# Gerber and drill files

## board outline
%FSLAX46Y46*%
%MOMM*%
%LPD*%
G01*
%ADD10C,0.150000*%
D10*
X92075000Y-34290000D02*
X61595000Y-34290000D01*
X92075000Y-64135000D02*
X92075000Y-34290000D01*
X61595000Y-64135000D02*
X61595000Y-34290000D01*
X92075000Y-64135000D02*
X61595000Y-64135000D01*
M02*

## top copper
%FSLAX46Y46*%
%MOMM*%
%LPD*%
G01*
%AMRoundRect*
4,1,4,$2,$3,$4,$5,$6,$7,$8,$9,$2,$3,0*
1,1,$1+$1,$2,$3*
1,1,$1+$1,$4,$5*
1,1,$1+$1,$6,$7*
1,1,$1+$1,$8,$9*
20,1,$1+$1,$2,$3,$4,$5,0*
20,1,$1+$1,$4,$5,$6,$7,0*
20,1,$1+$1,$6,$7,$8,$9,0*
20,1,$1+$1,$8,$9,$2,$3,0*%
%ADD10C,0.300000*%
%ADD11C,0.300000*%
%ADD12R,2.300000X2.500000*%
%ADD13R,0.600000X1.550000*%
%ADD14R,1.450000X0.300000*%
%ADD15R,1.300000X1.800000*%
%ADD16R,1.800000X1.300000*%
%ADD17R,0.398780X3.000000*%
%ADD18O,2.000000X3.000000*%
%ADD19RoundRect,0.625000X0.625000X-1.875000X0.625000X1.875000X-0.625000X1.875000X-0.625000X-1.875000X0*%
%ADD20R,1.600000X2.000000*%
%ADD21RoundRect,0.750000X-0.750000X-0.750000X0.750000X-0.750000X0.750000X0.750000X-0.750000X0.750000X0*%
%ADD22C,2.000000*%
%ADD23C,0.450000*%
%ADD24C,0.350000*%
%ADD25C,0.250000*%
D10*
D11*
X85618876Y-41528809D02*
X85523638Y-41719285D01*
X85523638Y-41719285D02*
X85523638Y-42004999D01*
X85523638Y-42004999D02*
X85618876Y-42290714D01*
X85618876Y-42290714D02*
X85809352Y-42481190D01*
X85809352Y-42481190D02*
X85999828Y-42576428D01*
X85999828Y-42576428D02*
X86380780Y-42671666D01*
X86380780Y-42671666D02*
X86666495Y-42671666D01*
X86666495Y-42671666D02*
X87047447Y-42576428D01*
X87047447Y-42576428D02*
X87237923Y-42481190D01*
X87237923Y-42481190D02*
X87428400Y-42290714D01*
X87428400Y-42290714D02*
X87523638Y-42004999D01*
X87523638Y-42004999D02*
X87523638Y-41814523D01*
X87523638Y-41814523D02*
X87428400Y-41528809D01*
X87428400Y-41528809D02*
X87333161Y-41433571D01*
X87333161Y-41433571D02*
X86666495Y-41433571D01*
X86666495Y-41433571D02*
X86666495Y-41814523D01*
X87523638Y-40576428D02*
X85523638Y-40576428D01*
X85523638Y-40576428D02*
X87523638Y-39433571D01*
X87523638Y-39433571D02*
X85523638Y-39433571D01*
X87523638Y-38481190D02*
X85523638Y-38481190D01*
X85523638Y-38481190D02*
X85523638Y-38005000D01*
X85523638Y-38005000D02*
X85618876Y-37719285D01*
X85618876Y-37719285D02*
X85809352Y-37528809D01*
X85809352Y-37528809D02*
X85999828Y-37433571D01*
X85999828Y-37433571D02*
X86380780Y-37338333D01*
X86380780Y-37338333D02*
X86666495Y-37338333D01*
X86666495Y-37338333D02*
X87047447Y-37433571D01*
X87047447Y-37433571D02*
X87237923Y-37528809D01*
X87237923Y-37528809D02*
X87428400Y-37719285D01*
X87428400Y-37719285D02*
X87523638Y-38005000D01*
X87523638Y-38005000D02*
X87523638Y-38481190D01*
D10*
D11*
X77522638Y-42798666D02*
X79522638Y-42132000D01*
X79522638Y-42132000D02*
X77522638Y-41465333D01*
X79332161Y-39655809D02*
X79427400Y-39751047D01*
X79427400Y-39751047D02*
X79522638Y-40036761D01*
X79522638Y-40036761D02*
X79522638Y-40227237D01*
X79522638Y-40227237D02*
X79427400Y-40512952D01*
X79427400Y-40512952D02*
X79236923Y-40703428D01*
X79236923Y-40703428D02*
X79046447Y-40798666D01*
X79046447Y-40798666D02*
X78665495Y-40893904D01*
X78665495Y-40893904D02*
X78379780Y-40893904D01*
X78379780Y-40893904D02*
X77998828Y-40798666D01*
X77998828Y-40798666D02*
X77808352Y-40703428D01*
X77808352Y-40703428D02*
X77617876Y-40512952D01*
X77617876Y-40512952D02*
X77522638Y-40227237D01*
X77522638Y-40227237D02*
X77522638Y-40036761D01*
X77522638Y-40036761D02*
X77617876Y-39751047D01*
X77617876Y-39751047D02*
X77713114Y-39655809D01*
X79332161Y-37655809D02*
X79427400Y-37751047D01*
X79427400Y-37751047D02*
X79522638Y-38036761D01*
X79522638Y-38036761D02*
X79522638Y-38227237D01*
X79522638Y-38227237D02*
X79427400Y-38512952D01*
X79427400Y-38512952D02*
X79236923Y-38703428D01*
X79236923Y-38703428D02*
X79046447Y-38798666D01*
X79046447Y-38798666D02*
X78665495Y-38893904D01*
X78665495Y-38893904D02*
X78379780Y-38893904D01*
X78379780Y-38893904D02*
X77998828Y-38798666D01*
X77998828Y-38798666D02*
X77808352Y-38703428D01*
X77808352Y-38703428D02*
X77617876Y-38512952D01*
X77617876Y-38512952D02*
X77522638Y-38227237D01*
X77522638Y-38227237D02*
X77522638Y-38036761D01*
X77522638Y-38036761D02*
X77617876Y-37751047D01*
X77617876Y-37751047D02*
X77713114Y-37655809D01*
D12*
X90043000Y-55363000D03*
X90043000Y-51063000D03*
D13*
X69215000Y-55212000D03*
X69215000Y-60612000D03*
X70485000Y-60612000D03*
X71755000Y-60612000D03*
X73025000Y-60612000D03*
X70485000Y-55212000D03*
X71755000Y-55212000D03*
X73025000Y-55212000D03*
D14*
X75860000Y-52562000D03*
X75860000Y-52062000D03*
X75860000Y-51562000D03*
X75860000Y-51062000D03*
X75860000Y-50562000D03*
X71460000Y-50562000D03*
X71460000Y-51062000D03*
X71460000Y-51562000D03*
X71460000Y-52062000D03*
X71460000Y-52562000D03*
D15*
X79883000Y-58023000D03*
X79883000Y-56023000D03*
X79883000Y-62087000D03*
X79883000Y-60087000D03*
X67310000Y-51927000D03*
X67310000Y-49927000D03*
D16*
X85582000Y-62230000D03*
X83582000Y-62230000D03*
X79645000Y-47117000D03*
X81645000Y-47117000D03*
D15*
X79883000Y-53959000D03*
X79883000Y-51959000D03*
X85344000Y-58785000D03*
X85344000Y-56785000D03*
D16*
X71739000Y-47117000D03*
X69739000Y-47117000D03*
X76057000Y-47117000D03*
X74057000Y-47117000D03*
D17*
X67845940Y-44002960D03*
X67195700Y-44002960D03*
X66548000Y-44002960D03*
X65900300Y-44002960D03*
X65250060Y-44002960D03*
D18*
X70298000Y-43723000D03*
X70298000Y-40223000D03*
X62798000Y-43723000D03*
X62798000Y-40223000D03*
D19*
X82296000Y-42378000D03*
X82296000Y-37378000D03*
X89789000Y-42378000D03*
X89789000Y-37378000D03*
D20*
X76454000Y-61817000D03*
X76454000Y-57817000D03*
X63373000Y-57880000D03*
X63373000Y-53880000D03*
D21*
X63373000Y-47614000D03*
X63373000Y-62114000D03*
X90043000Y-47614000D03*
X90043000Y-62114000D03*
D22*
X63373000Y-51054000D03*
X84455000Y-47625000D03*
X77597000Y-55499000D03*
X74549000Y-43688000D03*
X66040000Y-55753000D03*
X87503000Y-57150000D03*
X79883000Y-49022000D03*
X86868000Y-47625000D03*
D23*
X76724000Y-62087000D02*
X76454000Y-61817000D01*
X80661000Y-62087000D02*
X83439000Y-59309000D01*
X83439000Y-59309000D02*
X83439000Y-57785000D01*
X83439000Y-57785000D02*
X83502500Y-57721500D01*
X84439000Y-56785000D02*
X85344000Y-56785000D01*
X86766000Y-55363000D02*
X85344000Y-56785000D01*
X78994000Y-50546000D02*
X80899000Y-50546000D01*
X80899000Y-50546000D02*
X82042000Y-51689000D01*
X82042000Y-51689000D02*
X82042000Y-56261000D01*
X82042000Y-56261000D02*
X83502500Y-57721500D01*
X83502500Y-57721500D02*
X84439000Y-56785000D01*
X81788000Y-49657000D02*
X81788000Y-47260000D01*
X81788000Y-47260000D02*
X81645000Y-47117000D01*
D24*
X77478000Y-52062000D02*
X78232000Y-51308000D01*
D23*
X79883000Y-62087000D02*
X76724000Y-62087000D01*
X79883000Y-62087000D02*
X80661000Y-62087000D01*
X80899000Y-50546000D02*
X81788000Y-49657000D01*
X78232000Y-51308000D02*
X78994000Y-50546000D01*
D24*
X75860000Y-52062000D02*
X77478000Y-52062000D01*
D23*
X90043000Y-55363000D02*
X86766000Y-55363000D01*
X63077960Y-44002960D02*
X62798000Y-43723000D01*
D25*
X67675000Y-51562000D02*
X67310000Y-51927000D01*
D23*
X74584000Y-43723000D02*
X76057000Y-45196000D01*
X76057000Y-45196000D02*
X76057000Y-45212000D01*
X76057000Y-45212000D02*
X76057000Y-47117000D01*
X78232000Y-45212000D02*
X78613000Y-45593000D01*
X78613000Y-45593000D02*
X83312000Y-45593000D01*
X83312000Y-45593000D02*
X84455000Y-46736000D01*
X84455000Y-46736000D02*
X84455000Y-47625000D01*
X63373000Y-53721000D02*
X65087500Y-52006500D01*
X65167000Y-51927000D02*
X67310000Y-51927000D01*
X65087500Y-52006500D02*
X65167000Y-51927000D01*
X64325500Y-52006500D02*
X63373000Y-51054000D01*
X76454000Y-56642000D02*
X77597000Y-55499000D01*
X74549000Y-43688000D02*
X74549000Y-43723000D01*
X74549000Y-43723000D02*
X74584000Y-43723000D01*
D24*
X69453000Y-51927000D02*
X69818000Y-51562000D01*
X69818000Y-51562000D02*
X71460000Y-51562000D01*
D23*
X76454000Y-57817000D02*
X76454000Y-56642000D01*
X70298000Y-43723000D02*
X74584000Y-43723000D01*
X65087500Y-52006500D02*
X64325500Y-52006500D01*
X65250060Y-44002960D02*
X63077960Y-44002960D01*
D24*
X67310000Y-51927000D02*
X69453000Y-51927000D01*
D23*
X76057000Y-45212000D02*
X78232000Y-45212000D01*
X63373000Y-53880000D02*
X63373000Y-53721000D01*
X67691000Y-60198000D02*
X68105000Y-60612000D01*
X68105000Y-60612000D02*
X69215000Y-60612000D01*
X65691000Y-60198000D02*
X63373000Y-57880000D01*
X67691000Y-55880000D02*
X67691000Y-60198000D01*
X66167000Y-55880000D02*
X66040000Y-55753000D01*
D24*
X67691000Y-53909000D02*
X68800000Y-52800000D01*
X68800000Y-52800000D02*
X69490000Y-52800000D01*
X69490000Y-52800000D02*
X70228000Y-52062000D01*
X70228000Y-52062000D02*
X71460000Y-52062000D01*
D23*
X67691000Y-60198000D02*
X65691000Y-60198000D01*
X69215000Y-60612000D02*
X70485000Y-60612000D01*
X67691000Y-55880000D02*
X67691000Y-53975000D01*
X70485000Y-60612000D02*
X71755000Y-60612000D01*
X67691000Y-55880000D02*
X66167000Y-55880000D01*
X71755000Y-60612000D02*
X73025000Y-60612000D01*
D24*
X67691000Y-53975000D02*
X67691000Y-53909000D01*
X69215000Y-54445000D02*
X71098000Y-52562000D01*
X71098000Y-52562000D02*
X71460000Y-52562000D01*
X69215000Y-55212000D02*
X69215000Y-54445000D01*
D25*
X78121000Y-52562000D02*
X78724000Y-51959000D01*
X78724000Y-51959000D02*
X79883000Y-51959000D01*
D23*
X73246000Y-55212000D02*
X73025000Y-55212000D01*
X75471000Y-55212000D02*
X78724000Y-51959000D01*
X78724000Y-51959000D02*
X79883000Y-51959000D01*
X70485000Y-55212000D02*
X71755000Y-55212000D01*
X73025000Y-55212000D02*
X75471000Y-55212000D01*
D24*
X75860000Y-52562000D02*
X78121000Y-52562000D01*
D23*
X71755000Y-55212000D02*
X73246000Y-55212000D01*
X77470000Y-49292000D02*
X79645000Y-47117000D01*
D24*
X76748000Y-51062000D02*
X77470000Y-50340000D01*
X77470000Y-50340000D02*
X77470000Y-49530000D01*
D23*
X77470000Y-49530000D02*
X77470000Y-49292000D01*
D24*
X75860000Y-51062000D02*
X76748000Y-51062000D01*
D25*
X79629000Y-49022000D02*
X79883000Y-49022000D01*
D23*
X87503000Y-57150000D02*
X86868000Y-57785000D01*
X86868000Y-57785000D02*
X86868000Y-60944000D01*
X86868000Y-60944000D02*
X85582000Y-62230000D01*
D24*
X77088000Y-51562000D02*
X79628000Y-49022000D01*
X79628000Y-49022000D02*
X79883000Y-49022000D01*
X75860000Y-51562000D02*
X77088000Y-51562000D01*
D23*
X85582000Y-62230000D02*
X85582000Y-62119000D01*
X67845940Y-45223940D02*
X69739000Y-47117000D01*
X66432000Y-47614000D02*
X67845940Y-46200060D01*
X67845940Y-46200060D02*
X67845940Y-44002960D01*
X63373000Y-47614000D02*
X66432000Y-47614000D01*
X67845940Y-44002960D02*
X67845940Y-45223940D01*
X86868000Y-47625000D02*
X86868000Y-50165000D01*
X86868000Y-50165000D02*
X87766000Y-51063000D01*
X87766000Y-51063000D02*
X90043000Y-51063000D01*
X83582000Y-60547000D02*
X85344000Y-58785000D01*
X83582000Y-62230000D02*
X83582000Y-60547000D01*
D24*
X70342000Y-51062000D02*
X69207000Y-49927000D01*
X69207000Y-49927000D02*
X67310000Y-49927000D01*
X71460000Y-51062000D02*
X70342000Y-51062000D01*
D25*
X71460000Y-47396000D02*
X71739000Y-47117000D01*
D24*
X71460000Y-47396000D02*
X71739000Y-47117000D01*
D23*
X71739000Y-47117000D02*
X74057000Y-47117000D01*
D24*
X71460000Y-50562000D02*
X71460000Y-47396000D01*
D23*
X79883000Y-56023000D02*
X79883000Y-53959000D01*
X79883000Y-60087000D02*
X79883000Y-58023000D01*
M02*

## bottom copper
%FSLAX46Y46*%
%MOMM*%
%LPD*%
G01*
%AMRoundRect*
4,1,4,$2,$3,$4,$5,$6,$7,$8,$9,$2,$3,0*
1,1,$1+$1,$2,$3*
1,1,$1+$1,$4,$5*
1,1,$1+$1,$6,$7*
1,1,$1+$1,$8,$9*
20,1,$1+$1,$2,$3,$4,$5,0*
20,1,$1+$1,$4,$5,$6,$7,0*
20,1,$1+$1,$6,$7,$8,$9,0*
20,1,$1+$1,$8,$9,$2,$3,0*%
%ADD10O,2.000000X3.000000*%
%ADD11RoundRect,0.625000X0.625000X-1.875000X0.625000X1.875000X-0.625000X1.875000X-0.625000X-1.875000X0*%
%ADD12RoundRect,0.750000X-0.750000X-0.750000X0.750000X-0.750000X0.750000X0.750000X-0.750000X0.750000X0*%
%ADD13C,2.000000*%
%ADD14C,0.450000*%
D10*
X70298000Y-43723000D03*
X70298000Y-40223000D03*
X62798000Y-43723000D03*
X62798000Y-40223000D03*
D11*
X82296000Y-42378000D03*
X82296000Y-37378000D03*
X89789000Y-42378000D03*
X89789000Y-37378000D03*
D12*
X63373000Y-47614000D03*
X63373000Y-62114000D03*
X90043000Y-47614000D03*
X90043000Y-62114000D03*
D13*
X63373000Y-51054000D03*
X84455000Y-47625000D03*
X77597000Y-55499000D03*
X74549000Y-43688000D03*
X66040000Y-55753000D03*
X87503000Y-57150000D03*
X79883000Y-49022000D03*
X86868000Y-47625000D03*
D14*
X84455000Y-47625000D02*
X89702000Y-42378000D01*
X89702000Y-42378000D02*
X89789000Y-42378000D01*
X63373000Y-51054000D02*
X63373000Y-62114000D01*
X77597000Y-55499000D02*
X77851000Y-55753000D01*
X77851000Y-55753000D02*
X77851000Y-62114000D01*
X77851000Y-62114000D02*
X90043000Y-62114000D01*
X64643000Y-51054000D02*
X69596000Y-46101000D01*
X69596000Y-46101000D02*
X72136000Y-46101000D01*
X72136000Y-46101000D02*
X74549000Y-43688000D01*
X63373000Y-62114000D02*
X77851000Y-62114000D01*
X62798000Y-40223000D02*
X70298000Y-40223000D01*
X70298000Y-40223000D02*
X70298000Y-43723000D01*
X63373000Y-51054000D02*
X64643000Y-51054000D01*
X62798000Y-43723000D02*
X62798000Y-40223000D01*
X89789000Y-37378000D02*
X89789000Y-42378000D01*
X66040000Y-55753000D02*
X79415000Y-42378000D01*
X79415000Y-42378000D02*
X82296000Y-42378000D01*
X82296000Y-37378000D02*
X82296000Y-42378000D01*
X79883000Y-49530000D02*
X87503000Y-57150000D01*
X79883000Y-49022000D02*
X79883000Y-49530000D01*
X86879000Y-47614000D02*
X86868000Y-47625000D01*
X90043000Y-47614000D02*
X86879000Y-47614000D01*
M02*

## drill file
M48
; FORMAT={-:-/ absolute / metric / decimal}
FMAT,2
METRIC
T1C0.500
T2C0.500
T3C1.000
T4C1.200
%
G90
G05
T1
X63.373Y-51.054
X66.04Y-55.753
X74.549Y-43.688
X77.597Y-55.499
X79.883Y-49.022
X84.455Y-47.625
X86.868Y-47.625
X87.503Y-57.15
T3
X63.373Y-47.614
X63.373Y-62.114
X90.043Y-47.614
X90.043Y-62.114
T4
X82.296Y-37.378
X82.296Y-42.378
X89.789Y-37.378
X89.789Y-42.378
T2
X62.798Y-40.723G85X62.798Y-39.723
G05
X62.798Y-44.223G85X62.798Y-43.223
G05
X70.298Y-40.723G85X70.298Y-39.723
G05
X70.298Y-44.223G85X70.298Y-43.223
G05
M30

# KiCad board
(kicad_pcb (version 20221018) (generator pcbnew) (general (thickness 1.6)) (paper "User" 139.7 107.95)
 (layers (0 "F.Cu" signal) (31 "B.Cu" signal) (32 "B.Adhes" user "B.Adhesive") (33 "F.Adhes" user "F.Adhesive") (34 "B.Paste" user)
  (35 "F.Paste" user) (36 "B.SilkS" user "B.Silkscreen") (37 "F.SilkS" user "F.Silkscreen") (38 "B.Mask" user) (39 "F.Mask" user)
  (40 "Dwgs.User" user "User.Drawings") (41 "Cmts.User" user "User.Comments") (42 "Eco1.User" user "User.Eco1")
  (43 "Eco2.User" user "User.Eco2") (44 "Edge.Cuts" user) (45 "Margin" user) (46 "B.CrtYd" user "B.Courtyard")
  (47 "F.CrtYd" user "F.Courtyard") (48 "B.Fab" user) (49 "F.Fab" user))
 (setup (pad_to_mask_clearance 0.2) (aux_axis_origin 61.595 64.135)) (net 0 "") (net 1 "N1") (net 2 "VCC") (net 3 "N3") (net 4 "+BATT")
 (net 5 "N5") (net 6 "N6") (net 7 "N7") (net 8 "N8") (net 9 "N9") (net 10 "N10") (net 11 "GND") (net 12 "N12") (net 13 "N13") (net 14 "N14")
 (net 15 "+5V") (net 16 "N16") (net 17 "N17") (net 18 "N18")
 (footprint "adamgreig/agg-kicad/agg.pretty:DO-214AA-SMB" (layer "F.Cu") (at 90.043 53.213 90)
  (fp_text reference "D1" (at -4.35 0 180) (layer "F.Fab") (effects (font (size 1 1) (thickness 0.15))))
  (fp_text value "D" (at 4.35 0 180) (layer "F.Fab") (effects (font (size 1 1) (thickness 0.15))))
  (pad "1" smd rect (at -2.15 0 90) (size 2.5 2.3) (layers "F.Cu" "F.Paste" "F.Mask") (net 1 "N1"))
  (pad "2" smd rect (at 2.15 0 90) (size 2.5 2.3) (layers "F.Cu" "F.Paste" "F.Mask") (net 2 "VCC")))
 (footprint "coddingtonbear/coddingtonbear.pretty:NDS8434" (layer "F.Cu") (at 71.12 57.912 90) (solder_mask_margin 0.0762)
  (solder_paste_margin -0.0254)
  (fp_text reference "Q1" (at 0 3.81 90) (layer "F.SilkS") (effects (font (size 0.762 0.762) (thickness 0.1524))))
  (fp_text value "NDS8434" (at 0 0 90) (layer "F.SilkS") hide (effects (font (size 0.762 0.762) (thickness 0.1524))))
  (pad "1" smd rect (at 2.7 -1.905 90) (size 1.55 0.6) (layers "F.Cu" "F.Paste" "F.Mask") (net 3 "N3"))
  (pad "2" smd rect (at -2.7 -1.905 90) (size 1.55 0.6) (layers "F.Cu" "F.Paste" "F.Mask") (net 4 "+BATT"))
  (pad "2" smd rect (at -2.7 -0.635 90) (size 1.55 0.6) (layers "F.Cu" "F.Paste" "F.Mask") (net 4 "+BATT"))
  (pad "2" smd rect (at -2.7 0.635 90) (size 1.55 0.6) (layers "F.Cu" "F.Paste" "F.Mask") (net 4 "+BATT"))
  (pad "2" smd rect (at -2.7 1.905 90) (size 1.55 0.6) (layers "F.Cu" "F.Paste" "F.Mask") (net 4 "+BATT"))
  (pad "3" smd rect (at 2.7 -0.635 90) (size 1.55 0.6) (layers "F.Cu" "F.Paste" "F.Mask") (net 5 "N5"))
  (pad "3" smd rect (at 2.7 0.635 90) (size 1.55 0.6) (layers "F.Cu" "F.Paste" "F.Mask") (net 5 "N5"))
  (pad "3" smd rect (at 2.7 1.905 90) (size 1.55 0.6) (layers "F.Cu" "F.Paste" "F.Mask") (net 5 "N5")))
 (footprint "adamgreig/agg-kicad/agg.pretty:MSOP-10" (layer "F.Cu") (at 73.66 51.562 180)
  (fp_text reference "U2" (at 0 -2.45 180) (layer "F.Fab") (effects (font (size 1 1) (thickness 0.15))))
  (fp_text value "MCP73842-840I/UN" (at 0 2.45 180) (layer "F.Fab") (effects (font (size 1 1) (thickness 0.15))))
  (pad "1" smd rect (at -2.2 -1 180) (size 1.45 0.3) (layers "F.Cu" "F.Paste" "F.Mask") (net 5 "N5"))
  (pad "2" smd rect (at -2.2 -0.5 180) (size 1.45 0.3) (layers "F.Cu" "F.Paste" "F.Mask") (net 1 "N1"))
  (pad "3" smd rect (at -2.2 0 180) (size 1.45 0.3) (layers "F.Cu" "F.Paste" "F.Mask") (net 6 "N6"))
  (pad "4" smd rect (at -2.2 0.5 180) (size 1.45 0.3) (layers "F.Cu" "F.Paste" "F.Mask") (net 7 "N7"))
  (pad "5" smd rect (at -2.2 1 180) (size 1.45 0.3) (layers "F.Cu" "F.Paste" "F.Mask") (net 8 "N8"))
  (pad "6" smd rect (at 2.2 1 180) (size 1.45 0.3) (layers "F.Cu" "F.Paste" "F.Mask") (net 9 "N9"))
  (pad "7" smd rect (at 2.2 0.5 180) (size 1.45 0.3) (layers "F.Cu" "F.Paste" "F.Mask") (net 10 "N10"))
  (pad "8" smd rect (at 2.2 0 180) (size 1.45 0.3) (layers "F.Cu" "F.Paste" "F.Mask") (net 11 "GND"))
  (pad "9" smd rect (at 2.2 -0.5 180) (size 1.45 0.3) (layers "F.Cu" "F.Paste" "F.Mask") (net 4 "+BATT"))
  (pad "10" smd rect (at 2.2 -1 180) (size 1.45 0.3) (layers "F.Cu" "F.Paste" "F.Mask") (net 3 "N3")))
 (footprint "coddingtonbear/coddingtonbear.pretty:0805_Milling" (layer "F.Cu") (at 79.883 57.023 90)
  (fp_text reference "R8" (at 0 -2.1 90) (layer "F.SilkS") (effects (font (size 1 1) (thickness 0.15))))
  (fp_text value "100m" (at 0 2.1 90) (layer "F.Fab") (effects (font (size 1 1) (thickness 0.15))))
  (pad "1" smd rect (at -1 0 90) (size 1.8 1.3) (layers "F.Cu" "F.Paste" "F.Mask") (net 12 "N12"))
  (pad "2" smd rect (at 1 0 90) (size 1.8 1.3) (layers "F.Cu" "F.Paste" "F.Mask") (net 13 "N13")))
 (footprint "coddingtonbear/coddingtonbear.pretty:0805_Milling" (layer "F.Cu") (at 79.883 61.087 90)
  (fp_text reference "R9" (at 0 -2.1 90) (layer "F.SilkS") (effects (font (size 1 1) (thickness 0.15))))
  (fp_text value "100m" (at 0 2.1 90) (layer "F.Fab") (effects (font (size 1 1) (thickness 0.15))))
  (pad "1" smd rect (at -1 0 90) (size 1.8 1.3) (layers "F.Cu" "F.Paste" "F.Mask") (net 1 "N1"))
  (pad "2" smd rect (at 1 0 90) (size 1.8 1.3) (layers "F.Cu" "F.Paste" "F.Mask") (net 12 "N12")))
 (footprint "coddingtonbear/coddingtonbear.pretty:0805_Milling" (layer "F.Cu") (at 67.31 50.927 90)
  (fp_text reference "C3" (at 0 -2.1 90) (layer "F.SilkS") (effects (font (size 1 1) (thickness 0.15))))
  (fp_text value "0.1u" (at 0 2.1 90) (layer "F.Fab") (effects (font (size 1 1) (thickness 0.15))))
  (pad "1" smd rect (at -1 0 90) (size 1.8 1.3) (layers "F.Cu" "F.Paste" "F.Mask") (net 11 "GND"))
  (pad "2" smd rect (at 1 0 90) (size 1.8 1.3) (layers "F.Cu" "F.Paste" "F.Mask") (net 10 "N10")))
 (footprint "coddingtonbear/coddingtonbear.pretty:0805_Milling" (layer "F.Cu") (at 84.582 62.23 180)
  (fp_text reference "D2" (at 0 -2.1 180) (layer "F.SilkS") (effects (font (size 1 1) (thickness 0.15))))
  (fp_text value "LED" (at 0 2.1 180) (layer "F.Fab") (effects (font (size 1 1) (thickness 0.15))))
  (pad "1" smd rect (at -1 0 180) (size 1.8 1.3) (layers "F.Cu" "F.Paste" "F.Mask") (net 6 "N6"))
  (pad "2" smd rect (at 1 0 180) (size 1.8 1.3) (layers "F.Cu" "F.Paste" "F.Mask") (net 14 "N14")))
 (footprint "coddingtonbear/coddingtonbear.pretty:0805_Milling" (layer "F.Cu") (at 80.645 47.117)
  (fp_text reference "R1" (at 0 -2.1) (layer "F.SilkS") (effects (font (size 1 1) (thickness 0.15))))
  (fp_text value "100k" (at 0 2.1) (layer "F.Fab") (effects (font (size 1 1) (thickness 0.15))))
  (pad "1" smd rect (at -1 0) (size 1.8 1.3) (layers "F.Cu" "F.Paste" "F.Mask") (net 7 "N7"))
  (pad "2" smd rect (at 1 0) (size 1.8 1.3) (layers "F.Cu" "F.Paste" "F.Mask") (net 1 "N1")))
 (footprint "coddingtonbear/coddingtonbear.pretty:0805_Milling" (layer "F.Cu") (at 79.883 52.959 90)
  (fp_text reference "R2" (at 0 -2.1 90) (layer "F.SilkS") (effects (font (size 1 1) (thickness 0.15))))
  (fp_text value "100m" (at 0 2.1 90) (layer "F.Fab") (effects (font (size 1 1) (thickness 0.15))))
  (pad "1" smd rect (at -1 0 90) (size 1.8 1.3) (layers "F.Cu" "F.Paste" "F.Mask") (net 13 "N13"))
  (pad "2" smd rect (at 1 0 90) (size 1.8 1.3) (layers "F.Cu" "F.Paste" "F.Mask") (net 5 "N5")))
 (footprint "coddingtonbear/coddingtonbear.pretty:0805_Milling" (layer "F.Cu") (at 85.344 57.785 90)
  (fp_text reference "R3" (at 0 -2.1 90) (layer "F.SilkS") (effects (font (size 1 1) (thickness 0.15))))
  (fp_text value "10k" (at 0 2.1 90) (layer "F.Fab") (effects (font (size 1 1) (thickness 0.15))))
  (pad "1" smd rect (at -1 0 90) (size 1.8 1.3) (layers "F.Cu" "F.Paste" "F.Mask") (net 14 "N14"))
  (pad "2" smd rect (at 1 0 90) (size 1.8 1.3) (layers "F.Cu" "F.Paste" "F.Mask") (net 1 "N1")))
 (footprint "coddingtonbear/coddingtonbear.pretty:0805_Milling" (layer "F.Cu") (at 70.739 47.117 180)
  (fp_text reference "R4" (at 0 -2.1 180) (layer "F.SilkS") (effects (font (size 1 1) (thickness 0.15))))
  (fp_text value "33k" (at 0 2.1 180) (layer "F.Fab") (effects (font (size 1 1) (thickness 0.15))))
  (pad "1" smd rect (at -1 0 180) (size 1.8 1.3) (layers "F.Cu" "F.Paste" "F.Mask") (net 9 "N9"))
  (pad "2" smd rect (at 1 0 180) (size 1.8 1.3) (layers "F.Cu" "F.Paste" "F.Mask") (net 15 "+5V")))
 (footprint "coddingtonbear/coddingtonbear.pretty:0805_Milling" (layer "F.Cu") (at 75.057 47.117 180)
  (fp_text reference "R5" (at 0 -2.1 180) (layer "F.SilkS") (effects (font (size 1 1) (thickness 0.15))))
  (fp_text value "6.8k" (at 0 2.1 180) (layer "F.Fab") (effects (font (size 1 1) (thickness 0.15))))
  (pad "1" smd rect (at -1 0 180) (size 1.8 1.3) (layers "F.Cu" "F.Paste" "F.Mask") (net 11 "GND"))
  (pad "2" smd rect (at 1 0 180) (size 1.8 1.3) (layers "F.Cu" "F.Paste" "F.Mask") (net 9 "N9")))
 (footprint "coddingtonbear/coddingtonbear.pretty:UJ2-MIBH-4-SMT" (layer "F.Cu") (at 66.548 44.323 180)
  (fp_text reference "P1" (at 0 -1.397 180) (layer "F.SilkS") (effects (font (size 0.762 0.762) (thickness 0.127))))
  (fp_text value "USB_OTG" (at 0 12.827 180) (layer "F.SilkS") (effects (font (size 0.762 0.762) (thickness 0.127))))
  (pad "1" smd rect (at -1.29794 0.32004 180) (size 0.39878 3) (layers "F.Cu" "F.Paste" "F.Mask") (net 15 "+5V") (clearance 0.2032))
  (pad "2" smd rect (at -0.6477 0.32004 180) (size 0.39878 3) (layers "F.Cu" "F.Paste" "F.Mask") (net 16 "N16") (clearance 0.2032))
  (pad "3" smd rect (at 0 0.32004 180) (size 0.39878 3) (layers "F.Cu" "F.Paste" "F.Mask") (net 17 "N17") (clearance 0.2032))
  (pad "4" smd rect (at 0.6477 0.32004 180) (size 0.39878 3) (layers "F.Cu" "F.Paste" "F.Mask") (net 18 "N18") (clearance 0.2032))
  (pad "5" smd rect (at 1.29794 0.32004 180) (size 0.39878 3) (layers "F.Cu" "F.Paste" "F.Mask") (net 11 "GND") (clearance 0.2032))
  (pad "6" thru_hole oval (at -3.75 0.6 180) (size 2 3) (drill oval 0.5 1.5) (layers "*.Cu" "*.Mask") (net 11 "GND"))
  (pad "6" thru_hole oval (at -3.75 4.1 180) (size 2 3) (drill oval 0.5 1.5) (layers "*.Cu" "*.Mask") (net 11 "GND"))
  (pad "6" thru_hole oval (at 3.75 0.6 180) (size 2 3) (drill oval 0.5 1.5) (layers "*.Cu" "*.Mask") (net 11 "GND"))
  (pad "6" thru_hole oval (at 3.75 4.1 180) (size 2 3) (drill oval 0.5 1.5) (layers "*.Cu" "*.Mask") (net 11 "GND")))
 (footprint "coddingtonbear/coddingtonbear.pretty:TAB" (layer "F.Cu") (at 82.296 39.878 90)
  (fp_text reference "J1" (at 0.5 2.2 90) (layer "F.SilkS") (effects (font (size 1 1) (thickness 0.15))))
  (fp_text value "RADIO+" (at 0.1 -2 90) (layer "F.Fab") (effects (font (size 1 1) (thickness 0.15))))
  (pad "1" thru_hole roundrect (at -2.5 0 90) (size 5 2.5) (drill 1.2) (layers "*.Cu" "*.Mask") (roundrect_rratio 0.25) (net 4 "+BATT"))
  (pad "1" thru_hole roundrect (at 2.5 0 90) (size 5 2.5) (drill 1.2) (layers "*.Cu" "*.Mask") (roundrect_rratio 0.25) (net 4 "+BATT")))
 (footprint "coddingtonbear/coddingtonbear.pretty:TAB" (layer "F.Cu") (at 89.789 39.878 90)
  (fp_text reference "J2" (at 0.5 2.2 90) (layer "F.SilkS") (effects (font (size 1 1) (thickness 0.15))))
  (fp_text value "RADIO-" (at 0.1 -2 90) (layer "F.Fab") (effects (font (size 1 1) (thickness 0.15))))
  (pad "1" thru_hole roundrect (at -2.5 0 90) (size 5 2.5) (drill 1.2) (layers "*.Cu" "*.Mask") (roundrect_rratio 0.25) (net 11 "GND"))
  (pad "1" thru_hole roundrect (at 2.5 0 90) (size 5 2.5) (drill 1.2) (layers "*.Cu" "*.Mask") (roundrect_rratio 0.25) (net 11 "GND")))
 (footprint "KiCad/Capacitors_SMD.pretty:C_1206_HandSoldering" (layer "F.Cu") (at 76.454 59.817 90)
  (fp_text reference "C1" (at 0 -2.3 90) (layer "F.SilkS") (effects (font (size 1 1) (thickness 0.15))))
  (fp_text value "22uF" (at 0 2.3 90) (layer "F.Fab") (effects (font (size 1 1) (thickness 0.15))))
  (pad "1" smd rect (at -2 0 90) (size 2 1.6) (layers "F.Cu" "F.Paste" "F.Mask") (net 1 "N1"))
  (pad "2" smd rect (at 2 0 90) (size 2 1.6) (layers "F.Cu" "F.Paste" "F.Mask") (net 11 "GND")))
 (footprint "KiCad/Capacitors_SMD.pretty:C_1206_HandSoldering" (layer "F.Cu") (at 63.373 55.88 90)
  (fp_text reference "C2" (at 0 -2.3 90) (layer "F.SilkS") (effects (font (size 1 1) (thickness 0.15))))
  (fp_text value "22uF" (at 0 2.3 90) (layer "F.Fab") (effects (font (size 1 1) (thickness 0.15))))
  (pad "1" smd rect (at -2 0 90) (size 2 1.6) (layers "F.Cu" "F.Paste" "F.Mask") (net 4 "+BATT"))
  (pad "2" smd rect (at 2 0 90) (size 2 1.6) (layers "F.Cu" "F.Paste" "F.Mask") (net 11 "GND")))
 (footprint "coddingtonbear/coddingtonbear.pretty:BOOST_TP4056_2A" (layer "F.Cu") (at 76.708 54.864)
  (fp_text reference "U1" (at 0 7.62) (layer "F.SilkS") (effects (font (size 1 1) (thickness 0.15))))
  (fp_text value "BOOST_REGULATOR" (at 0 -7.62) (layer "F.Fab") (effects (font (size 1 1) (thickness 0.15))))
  (pad "1" thru_hole roundrect (at -13.335 -7.25) (size 3 3) (drill 1) (layers "*.Cu" "*.Mask") (roundrect_rratio 0.25) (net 15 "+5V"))
  (pad "2" thru_hole roundrect (at -13.335 7.25) (size 3 3) (drill 1) (layers "*.Cu" "*.Mask") (roundrect_rratio 0.25) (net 11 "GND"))
  (pad "3" thru_hole roundrect (at 13.335 -7.25) (size 3 3) (drill 1) (layers "*.Cu" "*.Mask") (roundrect_rratio 0.25) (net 2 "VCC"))
  (pad "4" thru_hole roundrect (at 13.335 7.25) (size 3 3) (drill 1) (layers "*.Cu" "*.Mask") (roundrect_rratio 0.25) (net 11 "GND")))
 (gr_line (start 92.075 34.29) (end 61.595 34.29) (stroke (width 0.15) (type solid)) (layer "Edge.Cuts"))
 (gr_line (start 92.075 64.135) (end 92.075 34.29) (stroke (width 0.15) (type solid)) (layer "Edge.Cuts"))
 (gr_line (start 61.595 64.135) (end 61.595 34.29) (stroke (width 0.15) (type solid)) (layer "Edge.Cuts"))
 (gr_line (start 92.075 64.135) (end 61.595 64.135) (stroke (width 0.15) (type solid)) (layer "Edge.Cuts"))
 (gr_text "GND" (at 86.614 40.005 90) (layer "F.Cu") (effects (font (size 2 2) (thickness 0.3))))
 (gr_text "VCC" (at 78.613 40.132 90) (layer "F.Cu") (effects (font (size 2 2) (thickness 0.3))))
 (segment (start 76.724 62.087) (end 76.454 61.817) (width 0.45) (layer "F.Cu") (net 1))
 (segment (start 80.661 62.087) (end 83.439 59.309) (width 0.45) (layer "F.Cu") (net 1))
 (segment (start 83.439 59.309) (end 83.439 57.785) (width 0.45) (layer "F.Cu") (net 1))
 (segment (start 83.439 57.785) (end 83.5025 57.7215) (width 0.45) (layer "F.Cu") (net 1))
 (segment (start 84.439 56.785) (end 85.344 56.785) (width 0.45) (layer "F.Cu") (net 1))
 (segment (start 86.766 55.363) (end 85.344 56.785) (width 0.45) (layer "F.Cu") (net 1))
 (segment (start 78.994 50.546) (end 80.899 50.546) (width 0.45) (layer "F.Cu") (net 1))
 (segment (start 80.899 50.546) (end 82.042 51.689) (width 0.45) (layer "F.Cu") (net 1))
 (segment (start 82.042 51.689) (end 82.042 56.261) (width 0.45) (layer "F.Cu") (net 1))
 (segment (start 82.042 56.261) (end 83.5025 57.7215) (width 0.45) (layer "F.Cu") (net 1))
 (segment (start 83.5025 57.7215) (end 84.439 56.785) (width 0.45) (layer "F.Cu") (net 1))
 (segment (start 81.788 49.657) (end 81.788 47.26) (width 0.45) (layer "F.Cu") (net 1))
 (segment (start 81.788 47.26) (end 81.645 47.117) (width 0.45) (layer "F.Cu") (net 1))
 (segment (start 77.478 52.062) (end 78.232 51.308) (width 0.35) (layer "F.Cu") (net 1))
 (segment (start 79.883 62.087) (end 76.724 62.087) (width 0.45) (layer "F.Cu") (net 1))
 (segment (start 79.883 62.087) (end 80.661 62.087) (width 0.45) (layer "F.Cu") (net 1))
 (segment (start 80.899 50.546) (end 81.788 49.657) (width 0.45) (layer "F.Cu") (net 1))
 (segment (start 78.232 51.308) (end 78.994 50.546) (width 0.45) (layer "F.Cu") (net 1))
 (segment (start 75.86 52.062) (end 77.478 52.062) (width 0.35) (layer "F.Cu") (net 1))
 (segment (start 90.043 55.363) (end 86.766 55.363) (width 0.45) (layer "F.Cu") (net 1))
 (segment (start 63.07796 44.00296) (end 62.798 43.723) (width 0.45) (layer "F.Cu") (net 11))
 (segment (start 67.675 51.562) (end 67.31 51.927) (width 0.25) (layer "F.Cu") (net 11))
 (segment (start 74.584 43.723) (end 76.057 45.196) (width 0.45) (layer "F.Cu") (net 11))
 (segment (start 76.057 45.196) (end 76.057 45.212) (width 0.45) (layer "F.Cu") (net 11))
 (segment (start 76.057 45.212) (end 76.057 47.117) (width 0.45) (layer "F.Cu") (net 11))
 (segment (start 78.232 45.212) (end 78.613 45.593) (width 0.45) (layer "F.Cu") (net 11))
 (segment (start 78.613 45.593) (end 83.312 45.593) (width 0.45) (layer "F.Cu") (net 11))
 (segment (start 83.312 45.593) (end 84.455 46.736) (width 0.45) (layer "F.Cu") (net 11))
 (segment (start 84.455 46.736) (end 84.455 47.625) (width 0.45) (layer "F.Cu") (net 11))
 (segment (start 63.373 53.721) (end 65.0875 52.0065) (width 0.45) (layer "F.Cu") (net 11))
 (segment (start 65.167 51.927) (end 67.31 51.927) (width 0.45) (layer "F.Cu") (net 11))
 (segment (start 65.0875 52.0065) (end 65.167 51.927) (width 0.45) (layer "F.Cu") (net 11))
 (segment (start 64.3255 52.0065) (end 63.373 51.054) (width 0.45) (layer "F.Cu") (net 11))
 (segment (start 76.454 56.642) (end 77.597 55.499) (width 0.45) (layer "F.Cu") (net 11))
 (segment (start 74.549 43.688) (end 74.549 43.723) (width 0.45) (layer "F.Cu") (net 11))
 (segment (start 74.549 43.723) (end 74.584 43.723) (width 0.45) (layer "F.Cu") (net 11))
 (segment (start 69.453 51.927) (end 69.818 51.562) (width 0.35) (layer "F.Cu") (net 11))
 (segment (start 69.818 51.562) (end 71.46 51.562) (width 0.35) (layer "F.Cu") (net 11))
 (segment (start 76.454 57.817) (end 76.454 56.642) (width 0.45) (layer "F.Cu") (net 11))
 (segment (start 70.298 43.723) (end 74.584 43.723) (width 0.45) (layer "F.Cu") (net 11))
 (segment (start 65.0875 52.0065) (end 64.3255 52.0065) (width 0.45) (layer "F.Cu") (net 11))
 (segment (start 65.25006 44.00296) (end 63.07796 44.00296) (width 0.45) (layer "F.Cu") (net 11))
 (segment (start 67.31 51.927) (end 69.453 51.927) (width 0.35) (layer "F.Cu") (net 11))
 (segment (start 76.057 45.212) (end 78.232 45.212) (width 0.45) (layer "F.Cu") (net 11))
 (segment (start 63.373 53.88) (end 63.373 53.721) (width 0.45) (layer "F.Cu") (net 11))
 (via (at 63.373 51.054) (size 2) (drill 0.5) (layers "F.Cu" "B.Cu") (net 11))
 (via (at 84.455 47.625) (size 2) (drill 0.5) (layers "F.Cu" "B.Cu") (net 11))
 (via (at 77.597 55.499) (size 2) (drill 0.5) (layers "F.Cu" "B.Cu") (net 11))
 (via (at 74.549 43.688) (size 2) (drill 0.5) (layers "F.Cu" "B.Cu") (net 11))
 (segment (start 84.455 47.625) (end 89.702 42.378) (width 0.45) (layer "B.Cu") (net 11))
 (segment (start 89.702 42.378) (end 89.789 42.378) (width 0.45) (layer "B.Cu") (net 11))
 (segment (start 63.373 51.054) (end 63.373 62.114) (width 0.45) (layer "B.Cu") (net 11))
 (segment (start 77.597 55.499) (end 77.851 55.753) (width 0.45) (layer "B.Cu") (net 11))
 (segment (start 77.851 55.753) (end 77.851 62.114) (width 0.45) (layer "B.Cu") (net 11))
 (segment (start 77.851 62.114) (end 90.043 62.114) (width 0.45) (layer "B.Cu") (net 11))
 (segment (start 64.643 51.054) (end 69.596 46.101) (width 0.45) (layer "B.Cu") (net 11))
 (segment (start 69.596 46.101) (end 72.136 46.101) (width 0.45) (layer "B.Cu") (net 11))
 (segment (start 72.136 46.101) (end 74.549 43.688) (width 0.45) (layer "B.Cu") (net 11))
 (segment (start 63.373 62.114) (end 77.851 62.114) (width 0.45) (layer "B.Cu") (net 11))
 (segment (start 62.798 40.223) (end 70.298 40.223) (width 0.45) (layer "B.Cu") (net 11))
 (segment (start 70.298 40.223) (end 70.298 43.723) (width 0.45) (layer "B.Cu") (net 11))
 (segment (start 63.373 51.054) (end 64.643 51.054) (width 0.45) (layer "B.Cu") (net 11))
 (segment (start 62.798 43.723) (end 62.798 40.223) (width 0.45) (layer "B.Cu") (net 11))
 (segment (start 89.789 37.378) (end 89.789 42.378) (width 0.45) (layer "B.Cu") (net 11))
 (segment (start 67.691 60.198) (end 68.105 60.612) (width 0.45) (layer "F.Cu") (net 4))
 (segment (start 68.105 60.612) (end 69.215 60.612) (width 0.45) (layer "F.Cu") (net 4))
 (segment (start 65.691 60.198) (end 63.373 57.88) (width 0.45) (layer "F.Cu") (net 4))
 (segment (start 67.691 55.88) (end 67.691 60.198) (width 0.45) (layer "F.Cu") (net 4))
 (segment (start 66.167 55.88) (end 66.04 55.753) (width 0.45) (layer "F.Cu") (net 4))
 (segment (start 67.691 53.909) (end 68.8 52.8) (width 0.35) (layer "F.Cu") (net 4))
 (segment (start 68.8 52.8) (end 69.49 52.8) (width 0.35) (layer "F.Cu") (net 4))
 (segment (start 69.49 52.8) (end 70.228 52.062) (width 0.35) (layer "F.Cu") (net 4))
 (segment (start 70.228 52.062) (end 71.46 52.062) (width 0.35) (layer "F.Cu") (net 4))
 (segment (start 67.691 60.198) (end 65.691 60.198) (width 0.45) (layer "F.Cu") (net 4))
 (segment (start 69.215 60.612) (end 70.485 60.612) (width 0.45) (layer "F.Cu") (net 4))
 (segment (start 67.691 55.88) (end 67.691 53.975) (width 0.45) (layer "F.Cu") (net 4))
 (segment (start 70.485 60.612) (end 71.755 60.612) (width 0.45) (layer "F.Cu") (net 4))
 (segment (start 67.691 55.88) (end 66.167 55.88) (width 0.45) (layer "F.Cu") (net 4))
 (segment (start 71.755 60.612) (end 73.025 60.612) (width 0.45) (layer "F.Cu") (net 4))
 (segment (start 67.691 53.975) (end 67.691 53.909) (width 0.35) (layer "F.Cu") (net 4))
 (via (at 66.04 55.753) (size 2) (drill 0.5) (layers "F.Cu" "B.Cu") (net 4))
 (segment (start 66.04 55.753) (end 79.415 42.378) (width 0.45) (layer "B.Cu") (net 4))
 (segment (start 79.415 42.378) (end 82.296 42.378) (width 0.45) (layer "B.Cu") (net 4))
 (segment (start 82.296 37.378) (end 82.296 42.378) (width 0.45) (layer "B.Cu") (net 4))
 (segment (start 69.215 54.445) (end 71.098 52.562) (width 0.35) (layer "F.Cu") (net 3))
 (segment (start 71.098 52.562) (end 71.46 52.562) (width 0.35) (layer "F.Cu") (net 3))
 (segment (start 69.215 55.212) (end 69.215 54.445) (width 0.35) (layer "F.Cu") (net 3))
 (segment (start 78.121 52.562) (end 78.724 51.959) (width 0.25) (layer "F.Cu") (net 5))
 (segment (start 78.724 51.959) (end 79.883 51.959) (width 0.25) (layer "F.Cu") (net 5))
 (segment (start 73.246 55.212) (end 73.025 55.212) (width 0.45) (layer "F.Cu") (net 5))
 (segment (start 75.471 55.212) (end 78.724 51.959) (width 0.45) (layer "F.Cu") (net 5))
 (segment (start 78.724 51.959) (end 79.883 51.959) (width 0.45) (layer "F.Cu") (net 5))
 (segment (start 70.485 55.212) (end 71.755 55.212) (width 0.45) (layer "F.Cu") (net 5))
 (segment (start 73.025 55.212) (end 75.471 55.212) (width 0.45) (layer "F.Cu") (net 5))
 (segment (start 75.86 52.562) (end 78.121 52.562) (width 0.35) (layer "F.Cu") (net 5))
 (segment (start 71.755 55.212) (end 73.246 55.212) (width 0.45) (layer "F.Cu") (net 5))
 (segment (start 77.47 49.292) (end 79.645 47.117) (width 0.45) (layer "F.Cu") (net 7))
 (segment (start 76.748 51.062) (end 77.47 50.34) (width 0.35) (layer "F.Cu") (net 7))
 (segment (start 77.47 50.34) (end 77.47 49.53) (width 0.35) (layer "F.Cu") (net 7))
 (segment (start 77.47 49.53) (end 77.47 49.292) (width 0.45) (layer "F.Cu") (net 7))
 (segment (start 75.86 51.062) (end 76.748 51.062) (width 0.35) (layer "F.Cu") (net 7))
 (segment (start 79.629 49.022) (end 79.883 49.022) (width 0.25) (layer "F.Cu") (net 6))
 (segment (start 87.503 57.15) (end 86.868 57.785) (width 0.45) (layer "F.Cu") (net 6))
 (segment (start 86.868 57.785) (end 86.868 60.944) (width 0.45) (layer "F.Cu") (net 6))
 (segment (start 86.868 60.944) (end 85.582 62.23) (width 0.45) (layer "F.Cu") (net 6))
 (segment (start 77.088 51.562) (end 79.628 49.022) (width 0.35) (layer "F.Cu") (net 6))
 (segment (start 79.628 49.022) (end 79.883 49.022) (width 0.35) (layer "F.Cu") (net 6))
 (segment (start 75.86 51.562) (end 77.088 51.562) (width 0.35) (layer "F.Cu") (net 6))
 (segment (start 85.582 62.23) (end 85.582 62.119) (width 0.45) (layer "F.Cu") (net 6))
 (via (at 87.503 57.15) (size 2) (drill 0.5) (layers "F.Cu" "B.Cu") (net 6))
 (via (at 79.883 49.022) (size 2) (drill 0.5) (layers "F.Cu" "B.Cu") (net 6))
 (segment (start 79.883 49.53) (end 87.503 57.15) (width 0.45) (layer "B.Cu") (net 6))
 (segment (start 79.883 49.022) (end 79.883 49.53) (width 0.45) (layer "B.Cu") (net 6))
 (segment (start 67.84594 45.22394) (end 69.739 47.117) (width 0.45) (layer "F.Cu") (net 15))
 (segment (start 66.432 47.614) (end 67.84594 46.20006) (width 0.45) (layer "F.Cu") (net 15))
 (segment (start 67.84594 46.20006) (end 67.84594 44.00296) (width 0.45) (layer "F.Cu") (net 15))
 (segment (start 63.373 47.614) (end 66.432 47.614) (width 0.45) (layer "F.Cu") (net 15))
 (segment (start 67.84594 44.00296) (end 67.84594 45.22394) (width 0.45) (layer "F.Cu") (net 15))
 (segment (start 86.868 47.625) (end 86.868 50.165) (width 0.45) (layer "F.Cu") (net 2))
 (segment (start 86.868 50.165) (end 87.766 51.063) (width 0.45) (layer "F.Cu") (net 2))
 (segment (start 87.766 51.063) (end 90.043 51.063) (width 0.45) (layer "F.Cu") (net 2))
 (via (at 86.868 47.625) (size 2) (drill 0.5) (layers "F.Cu" "B.Cu") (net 2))
 (segment (start 86.879 47.614) (end 86.868 47.625) (width 0.45) (layer "B.Cu") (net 2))
 (segment (start 90.043 47.614) (end 86.879 47.614) (width 0.45) (layer "B.Cu") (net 2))
 (segment (start 83.582 60.547) (end 85.344 58.785) (width 0.45) (layer "F.Cu") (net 14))
 (segment (start 83.582 62.23) (end 83.582 60.547) (width 0.45) (layer "F.Cu") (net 14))
 (segment (start 70.342 51.062) (end 69.207 49.927) (width 0.35) (layer "F.Cu") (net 10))
 (segment (start 69.207 49.927) (end 67.31 49.927) (width 0.35) (layer "F.Cu") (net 10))
 (segment (start 71.46 51.062) (end 70.342 51.062) (width 0.35) (layer "F.Cu") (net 10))
 (segment (start 71.46 47.396) (end 71.739 47.117) (width 0.25) (layer "F.Cu") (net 9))
 (segment (start 71.46 47.396) (end 71.739 47.117) (width 0.35) (layer "F.Cu") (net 9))
 (segment (start 71.739 47.117) (end 74.057 47.117) (width 0.45) (layer "F.Cu") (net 9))
 (segment (start 71.46 50.562) (end 71.46 47.396) (width 0.35) (layer "F.Cu") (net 9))
 (segment (start 79.883 56.023) (end 79.883 53.959) (width 0.45) (layer "F.Cu") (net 13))
 (segment (start 79.883 60.087) (end 79.883 58.023) (width 0.45) (layer "F.Cu") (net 12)))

